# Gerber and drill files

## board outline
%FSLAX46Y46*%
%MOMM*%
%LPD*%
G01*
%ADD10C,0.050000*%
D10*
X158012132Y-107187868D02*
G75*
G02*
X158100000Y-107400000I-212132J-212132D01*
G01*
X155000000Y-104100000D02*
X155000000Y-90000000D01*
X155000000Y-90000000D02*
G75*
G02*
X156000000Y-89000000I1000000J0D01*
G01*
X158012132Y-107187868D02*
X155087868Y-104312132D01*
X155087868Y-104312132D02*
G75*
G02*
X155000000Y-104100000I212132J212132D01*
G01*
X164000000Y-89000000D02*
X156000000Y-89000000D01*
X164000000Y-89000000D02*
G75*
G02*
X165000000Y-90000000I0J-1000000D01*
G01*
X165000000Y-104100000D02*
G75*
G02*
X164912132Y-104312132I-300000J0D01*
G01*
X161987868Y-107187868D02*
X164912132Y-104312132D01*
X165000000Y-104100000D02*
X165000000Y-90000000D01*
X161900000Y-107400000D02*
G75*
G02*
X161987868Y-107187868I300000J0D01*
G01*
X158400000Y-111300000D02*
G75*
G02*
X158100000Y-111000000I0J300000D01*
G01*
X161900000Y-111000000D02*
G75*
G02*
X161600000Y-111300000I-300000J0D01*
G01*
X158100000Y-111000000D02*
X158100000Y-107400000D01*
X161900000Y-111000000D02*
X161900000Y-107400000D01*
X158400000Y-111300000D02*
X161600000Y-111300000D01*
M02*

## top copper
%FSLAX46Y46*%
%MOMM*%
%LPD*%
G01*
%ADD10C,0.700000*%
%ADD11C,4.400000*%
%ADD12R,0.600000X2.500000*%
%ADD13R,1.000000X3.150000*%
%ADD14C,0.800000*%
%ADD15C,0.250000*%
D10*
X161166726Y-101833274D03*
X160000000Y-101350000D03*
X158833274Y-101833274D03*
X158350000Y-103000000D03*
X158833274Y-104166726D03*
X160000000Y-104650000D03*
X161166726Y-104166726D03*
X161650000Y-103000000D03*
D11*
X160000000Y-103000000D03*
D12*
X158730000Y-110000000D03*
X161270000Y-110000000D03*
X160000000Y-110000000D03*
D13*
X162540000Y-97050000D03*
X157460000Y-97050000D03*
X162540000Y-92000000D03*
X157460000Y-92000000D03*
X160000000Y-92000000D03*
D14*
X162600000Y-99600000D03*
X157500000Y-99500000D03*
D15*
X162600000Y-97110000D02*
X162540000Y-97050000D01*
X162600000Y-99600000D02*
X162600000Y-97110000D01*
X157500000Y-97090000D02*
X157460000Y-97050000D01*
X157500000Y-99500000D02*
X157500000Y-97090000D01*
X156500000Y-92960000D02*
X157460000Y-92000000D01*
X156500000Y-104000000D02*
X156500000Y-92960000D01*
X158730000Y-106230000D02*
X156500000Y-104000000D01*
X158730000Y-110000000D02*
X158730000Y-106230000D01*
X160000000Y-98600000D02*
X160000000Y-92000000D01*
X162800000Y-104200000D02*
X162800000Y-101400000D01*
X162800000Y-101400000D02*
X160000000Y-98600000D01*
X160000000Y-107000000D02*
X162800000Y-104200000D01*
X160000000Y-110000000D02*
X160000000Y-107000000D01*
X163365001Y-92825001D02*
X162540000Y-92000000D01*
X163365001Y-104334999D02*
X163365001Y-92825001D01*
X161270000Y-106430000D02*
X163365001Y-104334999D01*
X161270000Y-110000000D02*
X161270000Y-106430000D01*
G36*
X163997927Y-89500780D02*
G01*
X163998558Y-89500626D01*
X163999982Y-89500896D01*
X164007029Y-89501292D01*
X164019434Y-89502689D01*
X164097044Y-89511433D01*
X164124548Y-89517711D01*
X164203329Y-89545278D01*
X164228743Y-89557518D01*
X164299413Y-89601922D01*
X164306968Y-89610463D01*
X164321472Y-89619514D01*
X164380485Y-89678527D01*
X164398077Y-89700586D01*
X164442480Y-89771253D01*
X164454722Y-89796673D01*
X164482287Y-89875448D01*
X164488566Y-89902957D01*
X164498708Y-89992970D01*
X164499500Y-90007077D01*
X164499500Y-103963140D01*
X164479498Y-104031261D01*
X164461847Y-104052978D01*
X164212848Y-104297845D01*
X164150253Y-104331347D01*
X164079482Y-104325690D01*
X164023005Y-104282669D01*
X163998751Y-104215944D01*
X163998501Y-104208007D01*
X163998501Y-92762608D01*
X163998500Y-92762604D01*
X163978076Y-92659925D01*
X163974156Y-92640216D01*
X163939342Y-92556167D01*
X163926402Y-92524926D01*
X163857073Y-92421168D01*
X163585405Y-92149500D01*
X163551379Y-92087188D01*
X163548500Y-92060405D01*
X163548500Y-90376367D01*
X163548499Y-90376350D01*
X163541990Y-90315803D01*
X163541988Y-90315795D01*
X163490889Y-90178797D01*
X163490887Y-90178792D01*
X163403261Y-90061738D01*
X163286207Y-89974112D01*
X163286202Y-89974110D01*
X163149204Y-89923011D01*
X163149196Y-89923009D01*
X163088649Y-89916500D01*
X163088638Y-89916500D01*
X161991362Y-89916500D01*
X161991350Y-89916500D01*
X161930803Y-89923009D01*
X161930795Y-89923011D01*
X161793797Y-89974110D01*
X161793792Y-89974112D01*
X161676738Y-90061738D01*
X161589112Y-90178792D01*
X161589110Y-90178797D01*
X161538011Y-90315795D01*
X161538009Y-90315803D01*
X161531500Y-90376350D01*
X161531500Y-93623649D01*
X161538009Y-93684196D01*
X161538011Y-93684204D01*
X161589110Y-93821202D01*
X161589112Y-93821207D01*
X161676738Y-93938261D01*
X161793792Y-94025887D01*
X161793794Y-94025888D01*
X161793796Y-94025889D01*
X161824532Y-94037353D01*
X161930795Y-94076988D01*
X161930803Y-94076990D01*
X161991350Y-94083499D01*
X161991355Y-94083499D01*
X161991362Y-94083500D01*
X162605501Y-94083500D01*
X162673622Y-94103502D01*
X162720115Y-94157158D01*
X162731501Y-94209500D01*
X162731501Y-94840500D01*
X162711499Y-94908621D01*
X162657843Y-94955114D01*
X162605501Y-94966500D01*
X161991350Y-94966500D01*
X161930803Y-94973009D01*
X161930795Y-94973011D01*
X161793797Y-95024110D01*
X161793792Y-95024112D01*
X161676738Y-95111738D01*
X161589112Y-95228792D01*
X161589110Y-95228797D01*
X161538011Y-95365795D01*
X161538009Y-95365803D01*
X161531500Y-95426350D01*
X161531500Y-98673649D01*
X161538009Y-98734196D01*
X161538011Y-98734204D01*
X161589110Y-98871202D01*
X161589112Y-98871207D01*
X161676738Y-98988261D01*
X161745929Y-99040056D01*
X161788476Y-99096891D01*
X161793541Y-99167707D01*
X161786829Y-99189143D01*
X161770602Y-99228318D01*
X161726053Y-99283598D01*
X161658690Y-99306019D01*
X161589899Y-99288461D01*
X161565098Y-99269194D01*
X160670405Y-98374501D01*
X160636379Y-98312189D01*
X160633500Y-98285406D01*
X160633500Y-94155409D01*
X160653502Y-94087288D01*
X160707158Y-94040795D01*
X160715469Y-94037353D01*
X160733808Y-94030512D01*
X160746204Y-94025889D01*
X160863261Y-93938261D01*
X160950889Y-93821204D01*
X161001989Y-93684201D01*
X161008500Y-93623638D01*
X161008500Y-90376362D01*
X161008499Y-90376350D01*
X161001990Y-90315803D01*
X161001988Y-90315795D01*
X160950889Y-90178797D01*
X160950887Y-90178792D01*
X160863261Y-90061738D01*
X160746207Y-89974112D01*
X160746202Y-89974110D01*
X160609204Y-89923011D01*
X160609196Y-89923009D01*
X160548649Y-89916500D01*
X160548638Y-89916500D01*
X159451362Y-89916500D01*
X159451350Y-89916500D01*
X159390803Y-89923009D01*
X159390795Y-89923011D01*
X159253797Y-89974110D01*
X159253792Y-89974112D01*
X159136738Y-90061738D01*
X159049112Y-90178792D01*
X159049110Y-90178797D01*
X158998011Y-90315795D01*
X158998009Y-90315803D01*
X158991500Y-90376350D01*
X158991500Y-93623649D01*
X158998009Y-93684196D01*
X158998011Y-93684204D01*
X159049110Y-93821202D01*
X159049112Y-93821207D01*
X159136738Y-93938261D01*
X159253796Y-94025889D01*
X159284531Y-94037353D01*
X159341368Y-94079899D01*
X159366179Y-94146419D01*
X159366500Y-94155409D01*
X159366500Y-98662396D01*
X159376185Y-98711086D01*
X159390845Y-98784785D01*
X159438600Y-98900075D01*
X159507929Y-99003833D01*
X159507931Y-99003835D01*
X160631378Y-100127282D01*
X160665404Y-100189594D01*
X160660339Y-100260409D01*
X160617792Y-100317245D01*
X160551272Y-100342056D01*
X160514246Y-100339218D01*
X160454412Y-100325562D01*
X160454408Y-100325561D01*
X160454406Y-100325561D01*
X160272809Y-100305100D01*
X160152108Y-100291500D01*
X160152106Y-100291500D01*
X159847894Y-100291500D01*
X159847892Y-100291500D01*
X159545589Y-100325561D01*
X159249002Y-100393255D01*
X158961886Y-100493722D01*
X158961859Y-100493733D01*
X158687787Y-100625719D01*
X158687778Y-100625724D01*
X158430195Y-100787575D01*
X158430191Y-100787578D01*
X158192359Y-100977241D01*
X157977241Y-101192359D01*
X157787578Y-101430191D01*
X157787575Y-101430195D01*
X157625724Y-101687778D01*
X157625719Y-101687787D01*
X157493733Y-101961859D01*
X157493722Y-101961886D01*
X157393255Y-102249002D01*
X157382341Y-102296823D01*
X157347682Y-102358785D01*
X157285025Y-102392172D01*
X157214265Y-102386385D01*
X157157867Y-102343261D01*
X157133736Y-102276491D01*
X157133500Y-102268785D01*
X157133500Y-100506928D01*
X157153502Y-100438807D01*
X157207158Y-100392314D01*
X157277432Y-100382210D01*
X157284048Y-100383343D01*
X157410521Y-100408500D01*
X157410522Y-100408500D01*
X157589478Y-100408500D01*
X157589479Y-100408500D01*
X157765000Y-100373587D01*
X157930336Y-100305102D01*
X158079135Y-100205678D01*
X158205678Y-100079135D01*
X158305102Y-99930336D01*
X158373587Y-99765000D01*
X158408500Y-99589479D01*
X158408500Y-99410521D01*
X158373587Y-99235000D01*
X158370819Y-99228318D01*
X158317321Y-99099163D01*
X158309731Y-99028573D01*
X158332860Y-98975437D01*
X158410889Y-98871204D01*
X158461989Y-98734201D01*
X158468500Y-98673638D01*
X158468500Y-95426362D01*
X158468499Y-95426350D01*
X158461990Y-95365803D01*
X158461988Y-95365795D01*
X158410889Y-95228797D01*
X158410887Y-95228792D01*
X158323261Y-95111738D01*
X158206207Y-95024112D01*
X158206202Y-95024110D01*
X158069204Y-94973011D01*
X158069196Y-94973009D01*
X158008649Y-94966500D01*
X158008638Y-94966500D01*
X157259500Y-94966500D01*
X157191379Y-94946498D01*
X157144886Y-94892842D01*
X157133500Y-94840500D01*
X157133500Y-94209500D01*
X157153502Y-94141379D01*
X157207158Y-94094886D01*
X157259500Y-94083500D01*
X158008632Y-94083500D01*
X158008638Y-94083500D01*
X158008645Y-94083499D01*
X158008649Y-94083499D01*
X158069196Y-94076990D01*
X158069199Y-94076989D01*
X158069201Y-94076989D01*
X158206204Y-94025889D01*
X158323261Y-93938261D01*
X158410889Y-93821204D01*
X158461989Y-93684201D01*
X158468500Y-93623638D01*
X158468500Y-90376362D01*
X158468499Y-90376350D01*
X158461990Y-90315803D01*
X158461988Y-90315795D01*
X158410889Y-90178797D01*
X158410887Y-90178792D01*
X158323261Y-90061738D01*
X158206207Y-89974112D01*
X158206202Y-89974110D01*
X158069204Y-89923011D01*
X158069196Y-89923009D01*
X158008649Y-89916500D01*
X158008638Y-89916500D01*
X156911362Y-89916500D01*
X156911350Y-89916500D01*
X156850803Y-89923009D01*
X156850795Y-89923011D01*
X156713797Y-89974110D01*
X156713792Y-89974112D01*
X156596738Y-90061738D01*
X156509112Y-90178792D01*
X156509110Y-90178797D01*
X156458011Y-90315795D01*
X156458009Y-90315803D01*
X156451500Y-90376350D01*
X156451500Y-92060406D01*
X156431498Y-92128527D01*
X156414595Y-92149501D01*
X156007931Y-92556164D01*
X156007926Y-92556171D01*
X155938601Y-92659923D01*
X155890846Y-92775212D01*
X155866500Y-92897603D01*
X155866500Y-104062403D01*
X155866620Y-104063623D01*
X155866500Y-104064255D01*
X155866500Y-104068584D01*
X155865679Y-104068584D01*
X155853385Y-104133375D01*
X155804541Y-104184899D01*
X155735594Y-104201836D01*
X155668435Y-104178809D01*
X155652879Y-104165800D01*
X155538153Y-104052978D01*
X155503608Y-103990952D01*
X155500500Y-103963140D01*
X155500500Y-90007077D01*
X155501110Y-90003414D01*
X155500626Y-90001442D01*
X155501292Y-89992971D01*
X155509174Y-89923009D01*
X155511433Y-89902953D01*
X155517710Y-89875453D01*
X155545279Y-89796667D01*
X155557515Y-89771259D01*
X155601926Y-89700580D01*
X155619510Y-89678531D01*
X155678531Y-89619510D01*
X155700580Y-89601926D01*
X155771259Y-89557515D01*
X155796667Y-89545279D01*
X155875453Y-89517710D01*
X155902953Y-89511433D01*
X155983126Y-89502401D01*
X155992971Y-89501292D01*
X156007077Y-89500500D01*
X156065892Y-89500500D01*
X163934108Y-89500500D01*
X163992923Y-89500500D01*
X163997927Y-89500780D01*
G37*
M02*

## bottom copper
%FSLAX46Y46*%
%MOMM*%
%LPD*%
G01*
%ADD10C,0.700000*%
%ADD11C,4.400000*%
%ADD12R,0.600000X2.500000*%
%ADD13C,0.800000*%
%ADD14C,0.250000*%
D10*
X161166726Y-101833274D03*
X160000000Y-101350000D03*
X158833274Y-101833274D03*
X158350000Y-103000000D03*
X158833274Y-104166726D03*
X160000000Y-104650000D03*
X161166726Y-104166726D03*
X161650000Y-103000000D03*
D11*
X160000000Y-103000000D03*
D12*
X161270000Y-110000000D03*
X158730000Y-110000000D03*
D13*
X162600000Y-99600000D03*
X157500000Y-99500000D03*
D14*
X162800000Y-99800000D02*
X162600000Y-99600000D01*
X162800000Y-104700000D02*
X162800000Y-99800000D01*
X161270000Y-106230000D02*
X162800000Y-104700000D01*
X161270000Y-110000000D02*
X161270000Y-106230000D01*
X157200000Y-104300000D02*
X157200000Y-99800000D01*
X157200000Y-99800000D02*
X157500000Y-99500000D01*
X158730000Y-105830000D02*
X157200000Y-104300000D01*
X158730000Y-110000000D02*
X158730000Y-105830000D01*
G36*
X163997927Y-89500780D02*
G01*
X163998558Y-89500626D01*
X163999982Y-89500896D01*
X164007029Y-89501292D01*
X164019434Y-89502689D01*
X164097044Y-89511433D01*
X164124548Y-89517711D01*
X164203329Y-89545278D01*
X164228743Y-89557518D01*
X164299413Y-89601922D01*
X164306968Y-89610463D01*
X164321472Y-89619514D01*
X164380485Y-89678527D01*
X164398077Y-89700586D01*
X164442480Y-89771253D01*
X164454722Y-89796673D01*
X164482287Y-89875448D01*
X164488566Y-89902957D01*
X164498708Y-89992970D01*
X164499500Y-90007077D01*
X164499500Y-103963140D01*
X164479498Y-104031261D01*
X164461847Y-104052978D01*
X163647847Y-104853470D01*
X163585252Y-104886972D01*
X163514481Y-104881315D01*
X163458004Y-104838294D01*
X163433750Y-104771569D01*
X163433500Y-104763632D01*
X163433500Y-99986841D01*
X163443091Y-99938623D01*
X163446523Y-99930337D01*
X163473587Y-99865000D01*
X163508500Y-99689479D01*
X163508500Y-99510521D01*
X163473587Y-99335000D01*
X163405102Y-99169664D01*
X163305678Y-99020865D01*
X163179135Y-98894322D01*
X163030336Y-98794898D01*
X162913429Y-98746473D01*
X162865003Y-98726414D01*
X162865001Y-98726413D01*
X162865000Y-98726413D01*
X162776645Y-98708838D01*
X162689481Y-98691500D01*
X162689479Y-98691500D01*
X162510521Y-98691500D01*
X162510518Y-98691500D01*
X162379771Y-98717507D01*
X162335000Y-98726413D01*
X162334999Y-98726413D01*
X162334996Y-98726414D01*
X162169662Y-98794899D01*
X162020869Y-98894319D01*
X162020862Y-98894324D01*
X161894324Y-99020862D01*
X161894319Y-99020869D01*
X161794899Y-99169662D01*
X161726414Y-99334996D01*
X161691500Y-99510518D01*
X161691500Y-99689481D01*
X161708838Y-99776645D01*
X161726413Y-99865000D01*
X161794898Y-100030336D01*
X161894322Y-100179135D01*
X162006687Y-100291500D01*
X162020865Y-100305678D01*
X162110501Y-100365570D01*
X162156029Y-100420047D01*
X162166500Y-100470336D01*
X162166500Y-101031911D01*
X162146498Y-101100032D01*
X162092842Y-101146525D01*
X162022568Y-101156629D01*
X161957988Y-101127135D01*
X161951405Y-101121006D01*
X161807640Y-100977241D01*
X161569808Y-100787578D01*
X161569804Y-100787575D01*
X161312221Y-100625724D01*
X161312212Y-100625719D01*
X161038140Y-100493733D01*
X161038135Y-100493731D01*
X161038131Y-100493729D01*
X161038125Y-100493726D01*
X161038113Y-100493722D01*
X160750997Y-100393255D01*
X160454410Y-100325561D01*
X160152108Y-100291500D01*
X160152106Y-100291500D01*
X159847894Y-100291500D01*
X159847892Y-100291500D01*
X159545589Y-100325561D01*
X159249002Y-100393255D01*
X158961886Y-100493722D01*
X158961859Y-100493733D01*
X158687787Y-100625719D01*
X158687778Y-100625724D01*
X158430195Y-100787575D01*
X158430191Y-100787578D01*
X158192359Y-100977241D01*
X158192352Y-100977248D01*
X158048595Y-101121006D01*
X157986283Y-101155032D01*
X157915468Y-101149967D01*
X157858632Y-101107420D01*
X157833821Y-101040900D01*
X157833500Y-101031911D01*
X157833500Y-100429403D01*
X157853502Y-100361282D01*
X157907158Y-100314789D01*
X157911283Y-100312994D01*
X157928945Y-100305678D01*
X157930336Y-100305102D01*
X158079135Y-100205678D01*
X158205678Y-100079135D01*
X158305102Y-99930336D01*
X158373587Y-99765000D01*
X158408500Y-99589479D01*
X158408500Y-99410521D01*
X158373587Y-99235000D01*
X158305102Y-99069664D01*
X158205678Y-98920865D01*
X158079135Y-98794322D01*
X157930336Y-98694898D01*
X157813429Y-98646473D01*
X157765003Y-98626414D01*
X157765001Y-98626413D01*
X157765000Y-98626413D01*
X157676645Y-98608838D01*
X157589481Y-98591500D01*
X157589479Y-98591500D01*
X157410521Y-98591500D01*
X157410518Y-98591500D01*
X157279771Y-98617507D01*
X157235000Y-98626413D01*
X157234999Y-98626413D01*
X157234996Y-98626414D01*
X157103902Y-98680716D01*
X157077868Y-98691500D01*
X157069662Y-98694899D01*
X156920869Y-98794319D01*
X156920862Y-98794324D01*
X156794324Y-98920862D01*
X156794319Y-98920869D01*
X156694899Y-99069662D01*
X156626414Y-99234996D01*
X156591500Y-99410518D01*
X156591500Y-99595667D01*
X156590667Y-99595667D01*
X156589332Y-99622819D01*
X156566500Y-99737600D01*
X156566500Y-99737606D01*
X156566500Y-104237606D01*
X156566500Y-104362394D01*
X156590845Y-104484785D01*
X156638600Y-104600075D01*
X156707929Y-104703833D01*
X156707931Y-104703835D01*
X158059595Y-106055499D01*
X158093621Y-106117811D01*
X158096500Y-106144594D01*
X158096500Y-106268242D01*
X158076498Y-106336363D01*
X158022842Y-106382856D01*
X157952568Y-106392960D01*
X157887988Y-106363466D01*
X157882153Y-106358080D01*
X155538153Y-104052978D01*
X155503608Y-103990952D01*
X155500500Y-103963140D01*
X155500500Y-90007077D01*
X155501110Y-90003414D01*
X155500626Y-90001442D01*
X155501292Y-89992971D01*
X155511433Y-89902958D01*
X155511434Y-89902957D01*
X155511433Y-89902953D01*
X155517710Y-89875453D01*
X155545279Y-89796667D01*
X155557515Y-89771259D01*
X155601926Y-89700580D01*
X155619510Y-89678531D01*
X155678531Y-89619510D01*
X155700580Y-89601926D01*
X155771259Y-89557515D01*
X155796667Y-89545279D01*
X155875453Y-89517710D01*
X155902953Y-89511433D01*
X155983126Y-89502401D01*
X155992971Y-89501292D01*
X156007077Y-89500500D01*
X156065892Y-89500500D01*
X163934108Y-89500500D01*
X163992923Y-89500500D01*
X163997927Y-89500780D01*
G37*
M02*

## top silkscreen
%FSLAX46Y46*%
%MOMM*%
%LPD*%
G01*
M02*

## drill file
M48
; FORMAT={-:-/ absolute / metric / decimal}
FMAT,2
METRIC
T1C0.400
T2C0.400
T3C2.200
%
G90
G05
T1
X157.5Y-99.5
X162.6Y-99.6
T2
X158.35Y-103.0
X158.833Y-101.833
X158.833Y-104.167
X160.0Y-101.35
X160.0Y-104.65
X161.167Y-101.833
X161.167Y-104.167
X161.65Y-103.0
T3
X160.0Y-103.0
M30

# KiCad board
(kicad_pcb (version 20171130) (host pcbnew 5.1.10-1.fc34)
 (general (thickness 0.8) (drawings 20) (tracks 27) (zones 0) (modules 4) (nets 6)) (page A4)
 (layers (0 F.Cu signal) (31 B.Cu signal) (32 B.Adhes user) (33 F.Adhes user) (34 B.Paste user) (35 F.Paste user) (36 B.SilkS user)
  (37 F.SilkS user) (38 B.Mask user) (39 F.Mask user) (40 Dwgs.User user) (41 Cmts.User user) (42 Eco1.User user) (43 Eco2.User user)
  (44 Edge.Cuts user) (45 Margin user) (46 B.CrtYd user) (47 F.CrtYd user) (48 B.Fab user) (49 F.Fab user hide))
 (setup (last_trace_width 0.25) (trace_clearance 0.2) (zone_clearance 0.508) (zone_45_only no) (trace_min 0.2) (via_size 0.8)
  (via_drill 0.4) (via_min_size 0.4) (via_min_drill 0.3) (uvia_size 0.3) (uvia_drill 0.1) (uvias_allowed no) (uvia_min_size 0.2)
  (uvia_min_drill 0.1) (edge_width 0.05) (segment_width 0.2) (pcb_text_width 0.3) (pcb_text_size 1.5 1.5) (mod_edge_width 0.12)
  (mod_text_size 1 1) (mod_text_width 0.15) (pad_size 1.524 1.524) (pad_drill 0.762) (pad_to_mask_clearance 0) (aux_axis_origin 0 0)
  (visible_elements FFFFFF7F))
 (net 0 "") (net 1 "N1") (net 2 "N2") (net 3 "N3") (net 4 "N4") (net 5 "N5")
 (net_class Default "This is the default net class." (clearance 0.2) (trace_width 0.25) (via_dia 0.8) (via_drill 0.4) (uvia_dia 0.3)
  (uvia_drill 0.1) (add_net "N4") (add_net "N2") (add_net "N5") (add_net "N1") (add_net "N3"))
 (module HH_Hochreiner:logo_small (layer B.Cu) (at 160.1 92.8)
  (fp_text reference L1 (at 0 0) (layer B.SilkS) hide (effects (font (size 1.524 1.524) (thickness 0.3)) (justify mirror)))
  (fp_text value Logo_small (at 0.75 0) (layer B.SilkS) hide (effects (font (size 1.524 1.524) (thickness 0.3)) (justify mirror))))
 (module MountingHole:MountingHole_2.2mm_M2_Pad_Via (layer F.Cu) (at 160 103)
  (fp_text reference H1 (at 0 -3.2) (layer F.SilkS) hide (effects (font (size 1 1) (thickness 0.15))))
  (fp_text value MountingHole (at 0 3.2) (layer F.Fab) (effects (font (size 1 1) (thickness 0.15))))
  (pad 1 thru_hole circle (at 1.166726 -1.166726) (size 0.7 0.7) (drill 0.4) (layers *.Cu *.Mask))
  (pad 1 thru_hole circle (at 0 -1.65) (size 0.7 0.7) (drill 0.4) (layers *.Cu *.Mask))
  (pad 1 thru_hole circle (at -1.166726 -1.166726) (size 0.7 0.7) (drill 0.4) (layers *.Cu *.Mask))
  (pad 1 thru_hole circle (at -1.65 0) (size 0.7 0.7) (drill 0.4) (layers *.Cu *.Mask))
  (pad 1 thru_hole circle (at -1.166726 1.166726) (size 0.7 0.7) (drill 0.4) (layers *.Cu *.Mask))
  (pad 1 thru_hole circle (at 0 1.65) (size 0.7 0.7) (drill 0.4) (layers *.Cu *.Mask))
  (pad 1 thru_hole circle (at 1.166726 1.166726) (size 0.7 0.7) (drill 0.4) (layers *.Cu *.Mask))
  (pad 1 thru_hole circle (at 1.65 0) (size 0.7 0.7) (drill 0.4) (layers *.Cu *.Mask))
  (pad 1 thru_hole circle (at 0 0) (size 4.4 4.4) (drill 2.2) (layers *.Cu *.Mask)))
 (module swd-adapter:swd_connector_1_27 (layer F.Cu) (at 160 110)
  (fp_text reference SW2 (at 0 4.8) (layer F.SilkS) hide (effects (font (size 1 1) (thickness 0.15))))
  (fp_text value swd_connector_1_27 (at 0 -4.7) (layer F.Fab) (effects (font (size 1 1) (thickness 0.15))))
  (pad 5 smd rect (at 1.27 0) (size 0.6 2.5) (layers B.Cu B.Paste B.Mask) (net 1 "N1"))
  (pad 2 smd rect (at -1.27 0) (size 0.6 2.5) (layers F.Cu F.Paste F.Mask) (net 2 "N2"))
  (pad 6 smd rect (at 1.27 0) (size 0.6 2.5) (layers F.Cu F.Paste F.Mask) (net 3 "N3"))
  (pad 1 smd rect (at -1.27 0) (size 0.6 2.5) (layers B.Cu B.Paste B.Mask) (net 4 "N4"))
  (pad 4 smd rect (at 0 0) (size 0.6 2.5) (layers F.Cu F.Paste F.Mask) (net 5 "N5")))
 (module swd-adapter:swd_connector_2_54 (layer F.Cu) (at 160 94.525)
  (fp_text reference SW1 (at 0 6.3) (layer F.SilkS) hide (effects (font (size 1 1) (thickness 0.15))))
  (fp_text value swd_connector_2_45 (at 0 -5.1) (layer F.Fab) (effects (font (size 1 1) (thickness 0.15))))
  (pad 5 smd rect (at 2.54 2.525) (size 1 3.15) (layers F.Cu F.Paste F.Mask) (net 1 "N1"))
  (pad 1 smd rect (at -2.54 2.525) (size 1 3.15) (layers F.Cu F.Paste F.Mask) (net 4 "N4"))
  (pad 6 smd rect (at 2.54 -2.525) (size 1 3.15) (layers F.Cu F.Paste F.Mask) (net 3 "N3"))
  (pad 2 smd rect (at -2.54 -2.525) (size 1 3.15) (layers F.Cu F.Paste F.Mask) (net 2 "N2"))
  (pad 4 smd rect (at 0 -2.525) (size 1 3.15) (layers F.Cu F.Paste F.Mask) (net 5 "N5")))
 (gr_arc (start 157.8 107.4) (end 158.1 107.4) (angle -45) (layer Edge.Cuts) (width 0.05))
 (gr_line (start 155 104.1) (end 155 90) (layer Edge.Cuts) (width 0.05))
 (gr_arc (start 156 90) (end 155 90) (angle 90) (layer Edge.Cuts) (width 0.05))
 (gr_line (start 158.012132 107.187868) (end 155.087868 104.312132) (layer Edge.Cuts) (width 0.05))
 (gr_arc (start 155.3 104.1) (end 155 104.1) (angle -45) (layer Edge.Cuts) (width 0.05))
 (gr_line (start 164 89) (end 156 89) (layer Edge.Cuts) (width 0.05))
 (gr_arc (start 164 90) (end 165 90) (angle -90) (layer Edge.Cuts) (width 0.05))
 (gr_arc (start 164.7 104.1) (end 165 104.1) (angle 45) (layer Edge.Cuts) (width 0.05))
 (gr_line (start 161.987868 107.187868) (end 164.912132 104.312132) (layer Edge.Cuts) (width 0.05))
 (gr_line (start 165 104.1) (end 165 90) (layer Edge.Cuts) (width 0.05))
 (gr_arc (start 162.2 107.4) (end 161.9 107.4) (angle 45) (layer Edge.Cuts) (width 0.05))
 (gr_arc (start 158.4 111) (end 158.1 111) (angle -90) (layer Edge.Cuts) (width 0.05))
 (gr_arc (start 161.6 111) (end 161.6 111.3) (angle -90) (layer Edge.Cuts) (width 0.05))
 (gr_line (start 158.1 111) (end 158.1 107.4) (layer Edge.Cuts) (width 0.05))
 (gr_line (start 161.9 111) (end 161.9 107.4) (layer Edge.Cuts) (width 0.05))
 (gr_line (start 158.4 111.3) (end 161.6 111.3) (layer Edge.Cuts) (width 0.05))
 (via (at 162.6 99.6) (size 0.8) (drill 0.4) (layers F.Cu B.Cu) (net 1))
 (segment (start 162.6 97.11) (end 162.54 97.05) (width 0.25) (layer F.Cu) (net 1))
 (segment (start 162.6 99.6) (end 162.6 97.11) (width 0.25) (layer F.Cu) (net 1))
 (segment (start 162.8 99.8) (end 162.6 99.6) (width 0.25) (layer B.Cu) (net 1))
 (segment (start 162.8 104.7) (end 162.8 99.8) (width 0.25) (layer B.Cu) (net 1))
 (segment (start 161.27 106.23) (end 162.8 104.7) (width 0.25) (layer B.Cu) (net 1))
 (segment (start 161.27 110) (end 161.27 106.23) (width 0.25) (layer B.Cu) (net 1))
 (via (at 157.5 99.5) (size 0.8) (drill 0.4) (layers F.Cu B.Cu) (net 4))
 (segment (start 157.5 97.09) (end 157.46 97.05) (width 0.25) (layer F.Cu) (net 4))
 (segment (start 157.5 99.5) (end 157.5 97.09) (width 0.25) (layer F.Cu) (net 4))
 (segment (start 157.2 104.3) (end 157.2 99.8) (width 0.25) (layer B.Cu) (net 4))
 (segment (start 157.2 99.8) (end 157.5 99.5) (width 0.25) (layer B.Cu) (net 4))
 (segment (start 158.73 105.83) (end 157.2 104.3) (width 0.25) (layer B.Cu) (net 4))
 (segment (start 158.73 110) (end 158.73 105.83) (width 0.25) (layer B.Cu) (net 4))
 (segment (start 156.5 92.96) (end 157.46 92) (width 0.25) (layer F.Cu) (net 2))
 (segment (start 156.5 104) (end 156.5 92.96) (width 0.25) (layer F.Cu) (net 2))
 (segment (start 158.73 106.23) (end 156.5 104) (width 0.25) (layer F.Cu) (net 2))
 (segment (start 158.73 110) (end 158.73 106.23) (width 0.25) (layer F.Cu) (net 2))
 (segment (start 160 98.6) (end 160 92) (width 0.25) (layer F.Cu) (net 5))
 (segment (start 162.8 104.2) (end 162.8 101.4) (width 0.25) (layer F.Cu) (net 5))
 (segment (start 162.8 101.4) (end 160 98.6) (width 0.25) (layer F.Cu) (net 5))
 (segment (start 160 107) (end 162.8 104.2) (width 0.25) (layer F.Cu) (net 5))
 (segment (start 160 110) (end 160 107) (width 0.25) (layer F.Cu) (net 5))
 (segment (start 163.365001 92.825001) (end 162.54 92) (width 0.25) (layer F.Cu) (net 3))
 (segment (start 163.365001 104.334999) (end 163.365001 92.825001) (width 0.25) (layer F.Cu) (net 3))
 (segment (start 161.27 106.43) (end 163.365001 104.334999) (width 0.25) (layer F.Cu) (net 3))
 (segment (start 161.27 110) (end 161.27 106.43) (width 0.25) (layer F.Cu) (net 3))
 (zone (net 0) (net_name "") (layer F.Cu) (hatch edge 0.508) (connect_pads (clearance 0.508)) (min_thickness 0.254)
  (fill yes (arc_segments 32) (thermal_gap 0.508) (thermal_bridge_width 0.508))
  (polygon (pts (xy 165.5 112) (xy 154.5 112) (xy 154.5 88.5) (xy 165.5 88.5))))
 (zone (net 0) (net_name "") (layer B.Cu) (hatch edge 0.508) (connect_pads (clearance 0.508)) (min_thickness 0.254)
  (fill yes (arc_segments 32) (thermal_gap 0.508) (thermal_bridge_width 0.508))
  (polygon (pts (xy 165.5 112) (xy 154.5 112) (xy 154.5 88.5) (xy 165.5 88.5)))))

